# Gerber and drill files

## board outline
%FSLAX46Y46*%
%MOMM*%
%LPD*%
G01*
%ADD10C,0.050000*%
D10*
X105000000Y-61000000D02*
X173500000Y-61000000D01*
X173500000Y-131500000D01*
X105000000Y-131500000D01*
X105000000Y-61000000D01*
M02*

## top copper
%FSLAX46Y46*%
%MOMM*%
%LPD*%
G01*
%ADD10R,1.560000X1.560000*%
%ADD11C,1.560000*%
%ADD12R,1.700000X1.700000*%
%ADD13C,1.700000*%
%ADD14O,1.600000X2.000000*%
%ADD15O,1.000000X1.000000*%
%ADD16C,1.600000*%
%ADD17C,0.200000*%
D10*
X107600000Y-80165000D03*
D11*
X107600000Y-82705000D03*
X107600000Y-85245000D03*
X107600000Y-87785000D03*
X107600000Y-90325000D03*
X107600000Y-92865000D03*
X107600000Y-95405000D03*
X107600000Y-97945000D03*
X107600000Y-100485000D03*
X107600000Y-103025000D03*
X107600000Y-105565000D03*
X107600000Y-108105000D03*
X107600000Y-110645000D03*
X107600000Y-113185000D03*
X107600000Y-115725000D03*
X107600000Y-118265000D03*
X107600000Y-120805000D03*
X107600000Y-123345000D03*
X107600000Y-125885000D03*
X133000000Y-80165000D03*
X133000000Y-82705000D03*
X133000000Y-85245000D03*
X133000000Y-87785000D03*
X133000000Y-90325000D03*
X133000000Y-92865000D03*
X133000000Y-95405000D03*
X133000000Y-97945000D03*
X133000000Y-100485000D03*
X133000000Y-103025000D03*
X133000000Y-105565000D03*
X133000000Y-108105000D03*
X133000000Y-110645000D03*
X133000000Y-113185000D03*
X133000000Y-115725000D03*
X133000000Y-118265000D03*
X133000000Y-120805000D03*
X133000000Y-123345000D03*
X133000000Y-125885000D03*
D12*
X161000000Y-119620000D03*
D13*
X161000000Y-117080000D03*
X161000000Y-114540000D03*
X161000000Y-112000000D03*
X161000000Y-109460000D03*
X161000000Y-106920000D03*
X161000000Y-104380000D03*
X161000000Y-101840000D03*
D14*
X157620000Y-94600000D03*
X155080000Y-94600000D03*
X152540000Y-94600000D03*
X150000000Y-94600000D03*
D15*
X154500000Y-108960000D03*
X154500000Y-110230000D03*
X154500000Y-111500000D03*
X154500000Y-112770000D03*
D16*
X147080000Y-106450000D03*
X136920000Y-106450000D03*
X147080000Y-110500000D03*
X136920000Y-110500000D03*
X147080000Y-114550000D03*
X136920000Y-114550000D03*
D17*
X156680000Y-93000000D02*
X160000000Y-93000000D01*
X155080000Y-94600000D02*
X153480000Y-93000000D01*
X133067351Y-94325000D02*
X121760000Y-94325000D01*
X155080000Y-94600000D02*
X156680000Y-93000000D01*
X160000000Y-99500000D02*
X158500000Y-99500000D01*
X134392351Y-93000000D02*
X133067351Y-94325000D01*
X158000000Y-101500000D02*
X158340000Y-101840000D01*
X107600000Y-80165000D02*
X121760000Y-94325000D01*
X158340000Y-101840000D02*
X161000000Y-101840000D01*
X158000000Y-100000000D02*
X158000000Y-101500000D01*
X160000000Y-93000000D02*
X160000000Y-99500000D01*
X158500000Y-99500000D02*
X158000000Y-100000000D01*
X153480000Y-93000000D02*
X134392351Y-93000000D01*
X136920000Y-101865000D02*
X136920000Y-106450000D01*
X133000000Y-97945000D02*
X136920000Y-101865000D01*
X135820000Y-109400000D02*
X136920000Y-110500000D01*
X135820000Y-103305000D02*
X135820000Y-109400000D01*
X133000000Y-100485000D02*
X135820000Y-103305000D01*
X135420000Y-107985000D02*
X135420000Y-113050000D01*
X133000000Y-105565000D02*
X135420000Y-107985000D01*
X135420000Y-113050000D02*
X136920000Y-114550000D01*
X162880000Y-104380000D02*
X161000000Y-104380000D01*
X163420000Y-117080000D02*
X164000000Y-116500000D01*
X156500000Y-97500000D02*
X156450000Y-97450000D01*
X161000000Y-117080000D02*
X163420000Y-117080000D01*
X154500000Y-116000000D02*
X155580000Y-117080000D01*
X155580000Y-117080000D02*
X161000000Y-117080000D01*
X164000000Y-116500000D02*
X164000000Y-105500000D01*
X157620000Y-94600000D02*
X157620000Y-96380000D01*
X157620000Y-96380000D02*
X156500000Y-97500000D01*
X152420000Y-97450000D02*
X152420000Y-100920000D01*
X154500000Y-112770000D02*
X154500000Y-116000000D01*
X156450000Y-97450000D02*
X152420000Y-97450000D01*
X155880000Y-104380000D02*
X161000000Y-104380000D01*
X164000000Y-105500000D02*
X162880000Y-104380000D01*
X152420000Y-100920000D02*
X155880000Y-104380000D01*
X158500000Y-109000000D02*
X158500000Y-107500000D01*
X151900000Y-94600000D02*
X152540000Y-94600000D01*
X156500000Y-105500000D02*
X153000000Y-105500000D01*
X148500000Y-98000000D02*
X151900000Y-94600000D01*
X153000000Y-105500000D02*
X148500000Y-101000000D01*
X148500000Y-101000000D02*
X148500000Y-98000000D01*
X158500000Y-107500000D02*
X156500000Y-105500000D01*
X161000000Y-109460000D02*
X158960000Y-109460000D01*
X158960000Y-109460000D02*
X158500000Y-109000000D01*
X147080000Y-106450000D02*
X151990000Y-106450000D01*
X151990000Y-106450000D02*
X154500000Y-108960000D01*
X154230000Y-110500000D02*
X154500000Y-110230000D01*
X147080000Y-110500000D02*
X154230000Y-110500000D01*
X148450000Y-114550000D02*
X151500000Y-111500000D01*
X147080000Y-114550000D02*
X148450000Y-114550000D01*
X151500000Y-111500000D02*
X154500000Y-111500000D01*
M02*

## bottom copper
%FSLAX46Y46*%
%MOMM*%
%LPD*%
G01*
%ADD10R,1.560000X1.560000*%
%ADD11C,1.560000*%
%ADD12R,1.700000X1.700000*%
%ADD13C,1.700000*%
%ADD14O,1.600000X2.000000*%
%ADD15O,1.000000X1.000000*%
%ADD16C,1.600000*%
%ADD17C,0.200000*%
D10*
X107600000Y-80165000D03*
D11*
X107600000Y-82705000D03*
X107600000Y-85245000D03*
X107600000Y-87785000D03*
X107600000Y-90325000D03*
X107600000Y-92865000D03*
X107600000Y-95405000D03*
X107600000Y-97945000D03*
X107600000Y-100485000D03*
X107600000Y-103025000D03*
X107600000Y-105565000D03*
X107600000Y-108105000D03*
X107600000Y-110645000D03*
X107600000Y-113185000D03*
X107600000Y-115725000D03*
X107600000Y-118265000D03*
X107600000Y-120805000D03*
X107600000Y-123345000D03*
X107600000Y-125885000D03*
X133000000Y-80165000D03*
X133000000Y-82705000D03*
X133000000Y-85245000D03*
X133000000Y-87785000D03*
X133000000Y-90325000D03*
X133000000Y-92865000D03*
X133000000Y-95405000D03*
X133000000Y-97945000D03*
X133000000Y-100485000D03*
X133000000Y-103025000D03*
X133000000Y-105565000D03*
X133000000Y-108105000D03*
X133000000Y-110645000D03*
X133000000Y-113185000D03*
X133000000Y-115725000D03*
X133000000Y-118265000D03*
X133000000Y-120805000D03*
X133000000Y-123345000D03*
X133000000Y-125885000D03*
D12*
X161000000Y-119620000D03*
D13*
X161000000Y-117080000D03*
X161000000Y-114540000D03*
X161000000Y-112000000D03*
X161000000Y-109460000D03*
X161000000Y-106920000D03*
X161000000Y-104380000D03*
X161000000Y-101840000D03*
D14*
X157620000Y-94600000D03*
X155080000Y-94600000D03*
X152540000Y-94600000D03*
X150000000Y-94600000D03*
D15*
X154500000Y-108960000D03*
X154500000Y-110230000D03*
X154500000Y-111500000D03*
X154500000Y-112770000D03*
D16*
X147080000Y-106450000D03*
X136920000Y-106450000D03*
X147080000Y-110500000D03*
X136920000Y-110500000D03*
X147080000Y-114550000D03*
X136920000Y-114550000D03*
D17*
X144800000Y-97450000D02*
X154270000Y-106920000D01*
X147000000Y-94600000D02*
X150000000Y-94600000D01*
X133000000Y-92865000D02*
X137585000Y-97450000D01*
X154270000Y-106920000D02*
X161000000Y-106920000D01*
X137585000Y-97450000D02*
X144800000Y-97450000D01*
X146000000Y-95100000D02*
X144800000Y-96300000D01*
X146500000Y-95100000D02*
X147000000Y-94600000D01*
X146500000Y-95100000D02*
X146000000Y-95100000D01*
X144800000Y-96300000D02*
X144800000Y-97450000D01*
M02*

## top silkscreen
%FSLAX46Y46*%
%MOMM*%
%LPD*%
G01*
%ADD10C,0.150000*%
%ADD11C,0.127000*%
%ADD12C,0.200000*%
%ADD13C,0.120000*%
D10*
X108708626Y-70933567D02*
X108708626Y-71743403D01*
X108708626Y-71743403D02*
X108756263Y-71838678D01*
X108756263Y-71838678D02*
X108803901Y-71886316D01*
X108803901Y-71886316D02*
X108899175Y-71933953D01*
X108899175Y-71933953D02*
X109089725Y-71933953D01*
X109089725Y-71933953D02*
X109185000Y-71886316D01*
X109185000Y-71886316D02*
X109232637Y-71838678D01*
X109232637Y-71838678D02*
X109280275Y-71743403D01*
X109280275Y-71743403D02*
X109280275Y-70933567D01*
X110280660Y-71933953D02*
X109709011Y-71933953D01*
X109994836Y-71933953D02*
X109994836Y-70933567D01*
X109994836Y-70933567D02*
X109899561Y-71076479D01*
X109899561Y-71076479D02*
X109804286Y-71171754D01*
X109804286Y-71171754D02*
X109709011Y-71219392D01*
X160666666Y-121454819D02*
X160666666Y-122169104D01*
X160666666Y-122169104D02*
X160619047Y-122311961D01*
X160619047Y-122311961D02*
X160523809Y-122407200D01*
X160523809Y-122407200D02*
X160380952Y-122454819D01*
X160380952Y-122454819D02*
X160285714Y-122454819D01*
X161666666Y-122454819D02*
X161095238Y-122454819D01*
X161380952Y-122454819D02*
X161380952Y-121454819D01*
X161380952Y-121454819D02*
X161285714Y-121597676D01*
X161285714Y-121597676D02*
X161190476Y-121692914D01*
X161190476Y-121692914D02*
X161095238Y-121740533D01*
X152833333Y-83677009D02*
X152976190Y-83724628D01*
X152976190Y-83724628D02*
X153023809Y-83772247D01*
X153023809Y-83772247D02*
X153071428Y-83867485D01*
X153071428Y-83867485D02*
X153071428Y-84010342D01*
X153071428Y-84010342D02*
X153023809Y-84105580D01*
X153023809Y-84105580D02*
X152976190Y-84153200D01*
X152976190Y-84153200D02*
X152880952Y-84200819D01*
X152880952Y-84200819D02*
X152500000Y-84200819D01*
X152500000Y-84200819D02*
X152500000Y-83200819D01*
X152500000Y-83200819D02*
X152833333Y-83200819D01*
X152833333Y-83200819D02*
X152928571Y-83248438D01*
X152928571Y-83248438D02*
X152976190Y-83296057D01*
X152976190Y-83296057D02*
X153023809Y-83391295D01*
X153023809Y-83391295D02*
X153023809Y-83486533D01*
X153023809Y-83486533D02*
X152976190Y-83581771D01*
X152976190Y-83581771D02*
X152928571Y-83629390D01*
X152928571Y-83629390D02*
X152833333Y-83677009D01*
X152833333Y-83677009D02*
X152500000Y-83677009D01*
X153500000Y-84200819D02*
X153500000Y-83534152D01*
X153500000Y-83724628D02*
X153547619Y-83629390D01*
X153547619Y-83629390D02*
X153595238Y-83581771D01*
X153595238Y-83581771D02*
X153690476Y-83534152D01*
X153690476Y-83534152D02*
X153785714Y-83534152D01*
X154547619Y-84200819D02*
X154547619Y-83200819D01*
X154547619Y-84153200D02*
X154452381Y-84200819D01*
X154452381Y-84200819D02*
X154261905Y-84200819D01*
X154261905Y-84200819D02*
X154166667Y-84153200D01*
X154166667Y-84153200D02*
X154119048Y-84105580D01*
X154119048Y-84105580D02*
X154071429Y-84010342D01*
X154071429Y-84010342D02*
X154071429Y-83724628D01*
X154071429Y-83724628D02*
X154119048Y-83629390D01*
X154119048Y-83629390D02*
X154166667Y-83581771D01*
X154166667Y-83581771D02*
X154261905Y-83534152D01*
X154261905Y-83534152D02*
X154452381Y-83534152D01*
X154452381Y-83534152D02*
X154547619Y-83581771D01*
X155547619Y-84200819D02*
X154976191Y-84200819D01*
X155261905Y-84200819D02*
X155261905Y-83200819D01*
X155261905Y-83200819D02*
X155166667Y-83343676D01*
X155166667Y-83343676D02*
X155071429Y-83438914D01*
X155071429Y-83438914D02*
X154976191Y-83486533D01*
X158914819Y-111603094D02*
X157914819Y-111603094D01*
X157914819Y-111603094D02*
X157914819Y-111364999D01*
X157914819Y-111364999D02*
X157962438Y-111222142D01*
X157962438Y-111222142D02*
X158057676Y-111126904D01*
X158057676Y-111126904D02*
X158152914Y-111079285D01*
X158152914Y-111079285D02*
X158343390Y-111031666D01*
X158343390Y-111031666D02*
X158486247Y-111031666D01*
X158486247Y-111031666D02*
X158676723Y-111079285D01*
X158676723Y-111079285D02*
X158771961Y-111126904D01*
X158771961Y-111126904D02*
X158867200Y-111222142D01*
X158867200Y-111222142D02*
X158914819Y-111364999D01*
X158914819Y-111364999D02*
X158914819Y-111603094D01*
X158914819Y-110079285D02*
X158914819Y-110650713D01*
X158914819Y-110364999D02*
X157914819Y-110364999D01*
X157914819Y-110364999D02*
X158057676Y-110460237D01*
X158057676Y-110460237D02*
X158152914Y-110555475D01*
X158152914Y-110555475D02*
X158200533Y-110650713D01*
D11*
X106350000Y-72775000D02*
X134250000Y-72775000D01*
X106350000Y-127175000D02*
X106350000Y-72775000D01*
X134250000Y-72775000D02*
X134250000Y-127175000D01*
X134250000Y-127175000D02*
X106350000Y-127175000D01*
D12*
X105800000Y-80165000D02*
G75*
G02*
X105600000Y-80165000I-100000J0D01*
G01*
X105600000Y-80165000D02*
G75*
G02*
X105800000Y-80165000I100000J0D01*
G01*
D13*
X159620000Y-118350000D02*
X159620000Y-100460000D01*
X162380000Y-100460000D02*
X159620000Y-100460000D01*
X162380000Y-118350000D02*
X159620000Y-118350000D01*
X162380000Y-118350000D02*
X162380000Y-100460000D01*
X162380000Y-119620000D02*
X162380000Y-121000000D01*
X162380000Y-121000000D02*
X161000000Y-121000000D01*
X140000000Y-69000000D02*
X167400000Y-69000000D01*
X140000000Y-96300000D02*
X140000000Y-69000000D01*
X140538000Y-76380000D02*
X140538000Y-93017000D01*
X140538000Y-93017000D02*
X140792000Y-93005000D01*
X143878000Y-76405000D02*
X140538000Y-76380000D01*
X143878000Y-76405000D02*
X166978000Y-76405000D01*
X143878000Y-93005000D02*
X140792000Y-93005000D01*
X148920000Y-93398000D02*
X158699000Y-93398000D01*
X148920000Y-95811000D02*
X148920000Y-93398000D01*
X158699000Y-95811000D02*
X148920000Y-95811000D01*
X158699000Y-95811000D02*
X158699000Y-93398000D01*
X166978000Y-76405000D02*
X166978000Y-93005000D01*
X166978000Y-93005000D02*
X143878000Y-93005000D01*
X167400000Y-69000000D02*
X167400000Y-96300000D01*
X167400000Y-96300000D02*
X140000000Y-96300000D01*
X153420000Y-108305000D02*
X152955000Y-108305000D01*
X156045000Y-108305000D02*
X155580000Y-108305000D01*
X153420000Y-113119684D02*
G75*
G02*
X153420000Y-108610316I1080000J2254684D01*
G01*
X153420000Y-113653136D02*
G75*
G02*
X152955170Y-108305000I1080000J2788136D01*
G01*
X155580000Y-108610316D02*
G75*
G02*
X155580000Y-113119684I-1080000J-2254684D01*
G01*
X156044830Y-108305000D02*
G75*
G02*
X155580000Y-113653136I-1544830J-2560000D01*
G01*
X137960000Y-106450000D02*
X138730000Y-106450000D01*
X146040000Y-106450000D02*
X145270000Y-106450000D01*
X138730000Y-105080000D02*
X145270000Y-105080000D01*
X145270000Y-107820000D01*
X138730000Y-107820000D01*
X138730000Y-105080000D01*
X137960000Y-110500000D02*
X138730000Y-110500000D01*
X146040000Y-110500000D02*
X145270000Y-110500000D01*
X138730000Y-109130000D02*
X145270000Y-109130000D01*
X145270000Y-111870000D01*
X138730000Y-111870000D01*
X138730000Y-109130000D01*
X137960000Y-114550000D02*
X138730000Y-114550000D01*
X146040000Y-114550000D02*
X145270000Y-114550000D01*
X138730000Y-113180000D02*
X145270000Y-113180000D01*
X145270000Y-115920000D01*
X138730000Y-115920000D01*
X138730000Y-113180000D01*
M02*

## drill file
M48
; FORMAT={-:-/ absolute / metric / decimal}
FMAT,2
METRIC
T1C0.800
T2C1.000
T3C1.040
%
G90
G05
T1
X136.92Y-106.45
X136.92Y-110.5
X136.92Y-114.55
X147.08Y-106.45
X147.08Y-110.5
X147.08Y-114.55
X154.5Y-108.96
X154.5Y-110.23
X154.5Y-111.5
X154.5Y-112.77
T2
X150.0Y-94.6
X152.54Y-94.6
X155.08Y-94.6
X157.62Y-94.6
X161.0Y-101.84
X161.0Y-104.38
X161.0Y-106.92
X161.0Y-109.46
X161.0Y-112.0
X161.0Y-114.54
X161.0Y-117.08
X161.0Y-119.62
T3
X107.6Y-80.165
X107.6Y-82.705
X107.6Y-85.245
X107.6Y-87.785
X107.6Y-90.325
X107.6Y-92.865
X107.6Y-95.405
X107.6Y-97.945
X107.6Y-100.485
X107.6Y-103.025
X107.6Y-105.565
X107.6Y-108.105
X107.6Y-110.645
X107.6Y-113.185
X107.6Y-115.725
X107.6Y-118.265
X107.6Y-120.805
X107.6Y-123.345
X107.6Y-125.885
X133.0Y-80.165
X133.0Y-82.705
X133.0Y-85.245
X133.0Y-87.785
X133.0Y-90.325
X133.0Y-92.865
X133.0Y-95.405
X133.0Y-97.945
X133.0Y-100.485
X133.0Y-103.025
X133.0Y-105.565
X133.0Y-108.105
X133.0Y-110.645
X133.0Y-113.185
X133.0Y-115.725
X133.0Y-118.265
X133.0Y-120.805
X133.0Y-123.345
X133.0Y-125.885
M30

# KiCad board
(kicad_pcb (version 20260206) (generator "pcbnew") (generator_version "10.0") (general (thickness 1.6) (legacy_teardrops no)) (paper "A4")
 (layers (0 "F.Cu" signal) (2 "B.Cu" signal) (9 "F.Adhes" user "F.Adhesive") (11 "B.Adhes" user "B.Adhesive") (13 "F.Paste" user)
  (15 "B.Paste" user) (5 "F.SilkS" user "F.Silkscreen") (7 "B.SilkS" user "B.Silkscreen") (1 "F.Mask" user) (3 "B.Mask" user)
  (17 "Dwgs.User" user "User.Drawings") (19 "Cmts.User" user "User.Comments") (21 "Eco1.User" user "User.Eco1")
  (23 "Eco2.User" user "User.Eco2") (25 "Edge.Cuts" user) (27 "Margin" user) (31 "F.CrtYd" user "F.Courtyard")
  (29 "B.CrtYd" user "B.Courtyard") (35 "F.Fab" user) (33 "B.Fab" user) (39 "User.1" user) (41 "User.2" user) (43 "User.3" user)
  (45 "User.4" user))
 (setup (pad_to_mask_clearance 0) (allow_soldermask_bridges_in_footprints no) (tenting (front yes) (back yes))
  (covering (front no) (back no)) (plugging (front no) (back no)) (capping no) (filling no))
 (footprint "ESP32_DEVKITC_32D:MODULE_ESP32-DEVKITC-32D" (layer "F.Cu") (at 120.3 99.925)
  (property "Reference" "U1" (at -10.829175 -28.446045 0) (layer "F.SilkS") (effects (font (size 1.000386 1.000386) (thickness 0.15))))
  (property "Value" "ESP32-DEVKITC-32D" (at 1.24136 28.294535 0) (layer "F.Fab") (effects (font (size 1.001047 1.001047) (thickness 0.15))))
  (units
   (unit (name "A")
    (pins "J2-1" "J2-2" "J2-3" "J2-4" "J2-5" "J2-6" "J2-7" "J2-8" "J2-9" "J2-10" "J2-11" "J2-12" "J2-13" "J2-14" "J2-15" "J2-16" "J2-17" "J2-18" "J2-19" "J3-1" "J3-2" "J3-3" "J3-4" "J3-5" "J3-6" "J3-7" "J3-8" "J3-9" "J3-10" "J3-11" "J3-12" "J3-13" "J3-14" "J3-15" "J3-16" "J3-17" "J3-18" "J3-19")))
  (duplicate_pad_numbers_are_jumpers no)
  (fp_line (start -13.95 -27.15) (end 13.95 -27.15) (stroke (width 0.127) (type solid)) (layer "F.SilkS"))
  (fp_line (start -13.95 27.25) (end -13.95 -27.15) (stroke (width 0.127) (type solid)) (layer "F.SilkS"))
  (fp_line (start 13.95 -27.15) (end 13.95 27.25) (stroke (width 0.127) (type solid)) (layer "F.SilkS"))
  (fp_line (start 13.95 27.25) (end -13.95 27.25) (stroke (width 0.127) (type solid)) (layer "F.SilkS"))
  (fp_circle (center -14.6 -19.76) (end -14.5 -19.76) (stroke (width 0.2) (type solid)) (fill no) (layer "F.SilkS"))
  (pad "J2-1" thru_hole rect (at -12.7 -19.76) (size 1.56 1.56) (drill 1.04) (layers "*.Cu" "*.Mask") (remove_unused_layers no)
   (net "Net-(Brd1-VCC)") (solder_mask_margin 0.102))
  (pad "J2-2" thru_hole circle (at -12.7 -17.22) (size 1.56 1.56) (drill 1.04) (layers "*.Cu" "*.Mask") (remove_unused_layers no)
   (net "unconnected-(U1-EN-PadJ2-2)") (solder_mask_margin 0.102))
  (pad "J2-3" thru_hole circle (at -12.7 -14.68) (size 1.56 1.56) (drill 1.04) (layers "*.Cu" "*.Mask") (remove_unused_layers no)
   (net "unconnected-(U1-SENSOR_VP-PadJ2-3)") (solder_mask_margin 0.102))
  (pad "J2-4" thru_hole circle (at -12.7 -12.14) (size 1.56 1.56) (drill 1.04) (layers "*.Cu" "*.Mask") (remove_unused_layers no)
   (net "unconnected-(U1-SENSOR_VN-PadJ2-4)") (solder_mask_margin 0.102))
  (pad "J2-5" thru_hole circle (at -12.7 -9.6) (size 1.56 1.56) (drill 1.04) (layers "*.Cu" "*.Mask") (remove_unused_layers no)
   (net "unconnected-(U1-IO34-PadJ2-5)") (solder_mask_margin 0.102))
  (pad "J2-6" thru_hole circle (at -12.7 -7.06) (size 1.56 1.56) (drill 1.04) (layers "*.Cu" "*.Mask") (remove_unused_layers no)
   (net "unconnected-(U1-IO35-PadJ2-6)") (solder_mask_margin 0.102))
  (pad "J2-7" thru_hole circle (at -12.7 -4.52) (size 1.56 1.56) (drill 1.04) (layers "*.Cu" "*.Mask") (remove_unused_layers no)
   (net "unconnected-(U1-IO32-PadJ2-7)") (solder_mask_margin 0.102))
  (pad "J2-8" thru_hole circle (at -12.7 -1.98) (size 1.56 1.56) (drill 1.04) (layers "*.Cu" "*.Mask") (remove_unused_layers no)
   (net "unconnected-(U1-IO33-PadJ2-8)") (solder_mask_margin 0.102))
  (pad "J2-9" thru_hole circle (at -12.7 0.56) (size 1.56 1.56) (drill 1.04) (layers "*.Cu" "*.Mask") (remove_unused_layers no)
   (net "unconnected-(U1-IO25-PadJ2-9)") (solder_mask_margin 0.102))
  (pad "J2-10" thru_hole circle (at -12.7 3.1) (size 1.56 1.56) (drill 1.04) (layers "*.Cu" "*.Mask") (remove_unused_layers no)
   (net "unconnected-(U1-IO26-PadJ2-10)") (solder_mask_margin 0.102))
  (pad "J2-11" thru_hole circle (at -12.7 5.64) (size 1.56 1.56) (drill 1.04) (layers "*.Cu" "*.Mask") (remove_unused_layers no)
   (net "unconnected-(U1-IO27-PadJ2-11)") (solder_mask_margin 0.102))
  (pad "J2-12" thru_hole circle (at -12.7 8.18) (size 1.56 1.56) (drill 1.04) (layers "*.Cu" "*.Mask") (remove_unused_layers no)
   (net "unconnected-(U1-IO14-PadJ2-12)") (solder_mask_margin 0.102))
  (pad "J2-13" thru_hole circle (at -12.7 10.72) (size 1.56 1.56) (drill 1.04) (layers "*.Cu" "*.Mask") (remove_unused_layers no)
   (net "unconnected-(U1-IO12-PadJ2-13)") (solder_mask_margin 0.102))
  (pad "J2-14" thru_hole circle (at -12.7 13.26) (size 1.56 1.56) (drill 1.04) (layers "*.Cu" "*.Mask") (remove_unused_layers no)
   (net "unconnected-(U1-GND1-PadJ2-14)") (solder_mask_margin 0.102))
  (pad "J2-15" thru_hole circle (at -12.7 15.8) (size 1.56 1.56) (drill 1.04) (layers "*.Cu" "*.Mask") (remove_unused_layers no)
   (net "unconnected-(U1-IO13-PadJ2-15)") (solder_mask_margin 0.102))
  (pad "J2-16" thru_hole circle (at -12.7 18.34) (size 1.56 1.56) (drill 1.04) (layers "*.Cu" "*.Mask") (remove_unused_layers no)
   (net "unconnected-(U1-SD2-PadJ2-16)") (solder_mask_margin 0.102))
  (pad "J2-17" thru_hole circle (at -12.7 20.88) (size 1.56 1.56) (drill 1.04) (layers "*.Cu" "*.Mask") (remove_unused_layers no)
   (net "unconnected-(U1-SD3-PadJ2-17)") (solder_mask_margin 0.102))
  (pad "J2-18" thru_hole circle (at -12.7 23.42) (size 1.56 1.56) (drill 1.04) (layers "*.Cu" "*.Mask") (remove_unused_layers no)
   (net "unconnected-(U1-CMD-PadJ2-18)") (solder_mask_margin 0.102))
  (pad "J2-19" thru_hole circle (at -12.7 25.96) (size 1.56 1.56) (drill 1.04) (layers "*.Cu" "*.Mask") (remove_unused_layers no)
   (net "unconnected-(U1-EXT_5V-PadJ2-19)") (solder_mask_margin 0.102))
  (pad "J3-1" thru_hole circle (at 12.7 -19.76) (size 1.56 1.56) (drill 1.04) (layers "*.Cu" "*.Mask") (remove_unused_layers no)
   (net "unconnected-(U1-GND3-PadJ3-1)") (solder_mask_margin 0.102))
  (pad "J3-2" thru_hole circle (at 12.7 -17.22) (size 1.56 1.56) (drill 1.04) (layers "*.Cu" "*.Mask") (remove_unused_layers no)
   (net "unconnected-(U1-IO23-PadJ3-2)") (solder_mask_margin 0.102))
  (pad "J3-3" thru_hole circle (at 12.7 -14.68) (size 1.56 1.56) (drill 1.04) (layers "*.Cu" "*.Mask") (remove_unused_layers no)
   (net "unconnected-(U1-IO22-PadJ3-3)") (solder_mask_margin 0.102))
  (pad "J3-4" thru_hole circle (at 12.7 -12.14) (size 1.56 1.56) (drill 1.04) (layers "*.Cu" "*.Mask") (remove_unused_layers no)
   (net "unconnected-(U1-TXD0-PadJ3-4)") (solder_mask_margin 0.102))
  (pad "J3-5" thru_hole circle (at 12.7 -9.6) (size 1.56 1.56) (drill 1.04) (layers "*.Cu" "*.Mask") (remove_unused_layers no)
   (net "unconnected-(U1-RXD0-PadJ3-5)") (solder_mask_margin 0.102))
  (pad "J3-6" thru_hole circle (at 12.7 -7.06) (size 1.56 1.56) (drill 1.04) (layers "*.Cu" "*.Mask") (remove_unused_layers no) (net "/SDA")
   (solder_mask_margin 0.102))
  (pad "J3-7" thru_hole circle (at 12.7 -4.52) (size 1.56 1.56) (drill 1.04) (layers "*.Cu" "*.Mask") (remove_unused_layers no)
   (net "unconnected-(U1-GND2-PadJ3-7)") (solder_mask_margin 0.102))
  (pad "J3-8" thru_hole circle (at 12.7 -1.98) (size 1.56 1.56) (drill 1.04) (layers "*.Cu" "*.Mask") (remove_unused_layers no)
   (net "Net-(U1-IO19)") (solder_mask_margin 0.102))
  (pad "J3-9" thru_hole circle (at 12.7 0.56) (size 1.56 1.56) (drill 1.04) (layers "*.Cu" "*.Mask") (remove_unused_layers no)
   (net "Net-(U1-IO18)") (solder_mask_margin 0.102))
  (pad "J3-10" thru_hole circle (at 12.7 3.1) (size 1.56 1.56) (drill 1.04) (layers "*.Cu" "*.Mask") (remove_unused_layers no)
   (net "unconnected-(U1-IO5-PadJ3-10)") (solder_mask_margin 0.102))
  (pad "J3-11" thru_hole circle (at 12.7 5.64) (size 1.56 1.56) (drill 1.04) (layers "*.Cu" "*.Mask") (remove_unused_layers no)
   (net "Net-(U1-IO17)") (solder_mask_margin 0.102))
  (pad "J3-12" thru_hole circle (at 12.7 8.18) (size 1.56 1.56) (drill 1.04) (layers "*.Cu" "*.Mask") (remove_unused_layers no)
   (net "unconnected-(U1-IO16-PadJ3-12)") (solder_mask_margin 0.102))
  (pad "J3-13" thru_hole circle (at 12.7 10.72) (size 1.56 1.56) (drill 1.04) (layers "*.Cu" "*.Mask") (remove_unused_layers no)
   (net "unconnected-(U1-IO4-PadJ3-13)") (solder_mask_margin 0.102))
  (pad "J3-14" thru_hole circle (at 12.7 13.26) (size 1.56 1.56) (drill 1.04) (layers "*.Cu" "*.Mask") (remove_unused_layers no)
   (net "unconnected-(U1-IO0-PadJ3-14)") (solder_mask_margin 0.102))
  (pad "J3-15" thru_hole circle (at 12.7 15.8) (size 1.56 1.56) (drill 1.04) (layers "*.Cu" "*.Mask") (remove_unused_layers no)
   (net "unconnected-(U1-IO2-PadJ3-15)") (solder_mask_margin 0.102))
  (pad "J3-16" thru_hole circle (at 12.7 18.34) (size 1.56 1.56) (drill 1.04) (layers "*.Cu" "*.Mask") (remove_unused_layers no)
   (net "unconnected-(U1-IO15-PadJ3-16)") (solder_mask_margin 0.102))
  (pad "J3-17" thru_hole circle (at 12.7 20.88) (size 1.56 1.56) (drill 1.04) (layers "*.Cu" "*.Mask") (remove_unused_layers no)
   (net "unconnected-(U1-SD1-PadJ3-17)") (solder_mask_margin 0.102))
  (pad "J3-18" thru_hole circle (at 12.7 23.42) (size 1.56 1.56) (drill 1.04) (layers "*.Cu" "*.Mask") (remove_unused_layers no)
   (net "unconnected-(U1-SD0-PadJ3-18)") (solder_mask_margin 0.102))
  (pad "J3-19" thru_hole circle (at 12.7 25.96) (size 1.56 1.56) (drill 1.04) (layers "*.Cu" "*.Mask") (remove_unused_layers no)
   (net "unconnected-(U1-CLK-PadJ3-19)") (solder_mask_margin 0.102)))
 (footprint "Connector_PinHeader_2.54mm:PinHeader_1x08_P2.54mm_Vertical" (layer "F.Cu") (at 161 119.62 180)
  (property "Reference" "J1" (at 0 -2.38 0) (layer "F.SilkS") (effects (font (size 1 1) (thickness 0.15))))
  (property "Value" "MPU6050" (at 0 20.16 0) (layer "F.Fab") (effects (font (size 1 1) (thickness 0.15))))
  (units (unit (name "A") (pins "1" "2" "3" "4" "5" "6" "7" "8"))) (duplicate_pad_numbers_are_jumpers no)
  (fp_line (start 1.38 1.27) (end 1.38 19.16) (stroke (width 0.12) (type solid)) (layer "F.SilkS"))
  (fp_line (start -1.38 19.16) (end 1.38 19.16) (stroke (width 0.12) (type solid)) (layer "F.SilkS"))
  (fp_line (start -1.38 1.27) (end 1.38 1.27) (stroke (width 0.12) (type solid)) (layer "F.SilkS"))
  (fp_line (start -1.38 1.27) (end -1.38 19.16) (stroke (width 0.12) (type solid)) (layer "F.SilkS"))
  (fp_line (start -1.38 0) (end -1.38 -1.38) (stroke (width 0.12) (type solid)) (layer "F.SilkS"))
  (fp_line (start -1.38 -1.38) (end 0 -1.38) (stroke (width 0.12) (type solid)) (layer "F.SilkS"))
  (pad "1" thru_hole rect (at 0 0 180) (size 1.7 1.7) (drill 1) (layers "*.Cu" "*.Mask") (remove_unused_layers no)
   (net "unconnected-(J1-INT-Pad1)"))
  (pad "2" thru_hole circle (at 0 2.54 180) (size 1.7 1.7) (drill 1) (layers "*.Cu" "*.Mask") (remove_unused_layers no) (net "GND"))
  (pad "3" thru_hole circle (at 0 5.08 180) (size 1.7 1.7) (drill 1) (layers "*.Cu" "*.Mask") (remove_unused_layers no)
   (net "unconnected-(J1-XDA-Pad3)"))
  (pad "4" thru_hole circle (at 0 7.62 180) (size 1.7 1.7) (drill 1) (layers "*.Cu" "*.Mask") (remove_unused_layers no)
   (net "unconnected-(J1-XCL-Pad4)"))
  (pad "5" thru_hole circle (at 0 10.16 180) (size 1.7 1.7) (drill 1) (layers "*.Cu" "*.Mask") (remove_unused_layers no) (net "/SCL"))
  (pad "6" thru_hole circle (at 0 12.7 180) (size 1.7 1.7) (drill 1) (layers "*.Cu" "*.Mask") (remove_unused_layers no) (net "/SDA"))
  (pad "7" thru_hole circle (at 0 15.24 180) (size 1.7 1.7) (drill 1) (layers "*.Cu" "*.Mask") (remove_unused_layers no) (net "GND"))
  (pad "8" thru_hole circle (at 0 17.78 180) (size 1.7 1.7) (drill 1) (layers "*.Cu" "*.Mask") (remove_unused_layers no)
   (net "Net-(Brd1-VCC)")))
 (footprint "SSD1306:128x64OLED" (layer "F.Cu") (at 154 84 180)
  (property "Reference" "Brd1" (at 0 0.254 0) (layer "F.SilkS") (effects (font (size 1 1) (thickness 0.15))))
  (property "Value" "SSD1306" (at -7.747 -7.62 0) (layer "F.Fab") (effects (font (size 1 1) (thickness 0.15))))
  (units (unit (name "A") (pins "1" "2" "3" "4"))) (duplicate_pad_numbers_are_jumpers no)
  (fp_line (start 14 15) (end -13.4 15) (stroke (width 0.12) (type solid)) (layer "F.SilkS"))
  (fp_line (start 14 -12.3) (end 14 15) (stroke (width 0.12) (type solid)) (layer "F.SilkS"))
  (fp_line (start 13.462 7.62) (end 13.462 -9.017) (stroke (width 0.12) (type solid)) (layer "F.SilkS"))
  (fp_line (start 13.462 -9.017) (end 13.208 -9.005) (stroke (width 0.12) (type solid)) (layer "F.SilkS"))
  (fp_line (start 10.122 7.595) (end 13.462 7.62) (stroke (width 0.12) (type solid)) (layer "F.SilkS"))
  (fp_line (start 10.122 7.595) (end -12.978 7.595) (stroke (width 0.12) (type solid)) (layer "F.SilkS"))
  (fp_line (start 10.122 -9.005) (end 13.208 -9.005) (stroke (width 0.12) (type solid)) (layer "F.SilkS"))
  (fp_line (start 5.08 -9.398) (end -4.699 -9.398) (stroke (width 0.12) (type solid)) (layer "F.SilkS"))
  (fp_line (start 5.08 -11.811) (end 5.08 -9.398) (stroke (width 0.12) (type solid)) (layer "F.SilkS"))
  (fp_line (start -4.699 -11.811) (end 5.08 -11.811) (stroke (width 0.12) (type solid)) (layer "F.SilkS"))
  (fp_line (start -4.699 -11.811) (end -4.699 -9.398) (stroke (width 0.12) (type solid)) (layer "F.SilkS"))
  (fp_line (start -12.978 7.595) (end -12.978 -9.005) (stroke (width 0.12) (type solid)) (layer "F.SilkS"))
  (fp_line (start -12.978 -9.005) (end 10.122 -9.005) (stroke (width 0.12) (type solid)) (layer "F.SilkS"))
  (fp_line (start -13.4 15) (end -13.4 -12.3) (stroke (width 0.12) (type solid)) (layer "F.SilkS"))
  (fp_line (start -13.4 -12.3) (end 14 -12.3) (stroke (width 0.12) (type solid)) (layer "F.SilkS"))
  (pad "1" thru_hole oval (at -3.62 -10.6 270) (size 2 1.6) (drill 1) (layers "*.Cu" "*.Mask") (remove_unused_layers no) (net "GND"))
  (pad "2" thru_hole oval (at -1.08 -10.6 270) (size 2 1.6) (drill 1) (layers "*.Cu" "*.Mask") (remove_unused_layers no)
   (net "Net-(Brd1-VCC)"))
  (pad "3" thru_hole oval (at 1.46 -10.6 270) (size 2 1.6) (drill 1) (layers "*.Cu" "*.Mask") (remove_unused_layers no) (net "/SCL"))
  (pad "4" thru_hole oval (at 4 -10.6 270) (size 2 1.6) (drill 1) (layers "*.Cu" "*.Mask") (remove_unused_layers no) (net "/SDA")))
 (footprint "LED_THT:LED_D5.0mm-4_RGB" (layer "F.Cu") (at 154.5 108.96 -90)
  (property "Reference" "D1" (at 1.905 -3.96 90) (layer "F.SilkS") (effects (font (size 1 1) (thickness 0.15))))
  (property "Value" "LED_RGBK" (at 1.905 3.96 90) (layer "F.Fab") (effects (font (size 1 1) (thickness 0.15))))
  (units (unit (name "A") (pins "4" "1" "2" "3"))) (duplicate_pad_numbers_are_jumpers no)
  (fp_line (start -0.655 1.08) (end -0.655 1.545) (stroke (width 0.12) (type solid)) (layer "F.SilkS"))
  (fp_line (start -0.655 -1.545) (end -0.655 -1.08) (stroke (width 0.12) (type solid)) (layer "F.SilkS"))
  (fp_arc (start 4.159684 1.08) (mid 1.905 2.5) (end -0.349684 1.08) (stroke (width 0.12) (type solid)) (layer "F.SilkS"))
  (fp_arc (start 4.693136 1.08) (mid 2.163898 2.97877) (end -0.655 1.54483) (stroke (width 0.12) (type solid)) (layer "F.SilkS"))
  (fp_arc (start -0.349684 -1.08) (mid 1.905 -2.5) (end 4.159684 -1.08) (stroke (width 0.12) (type solid)) (layer "F.SilkS"))
  (fp_arc (start -0.655 -1.54483) (mid 2.163898 -2.97877) (end 4.693136 -1.08) (stroke (width 0.12) (type solid)) (layer "F.SilkS"))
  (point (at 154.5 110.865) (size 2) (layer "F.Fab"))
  (pad "1" thru_hole oval (at 0 0 270) (size 1 1) (drill 0.8) (layers "*.Cu" "*.Mask") (remove_unused_layers no) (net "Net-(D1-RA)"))
  (pad "2" thru_hole oval (at 1.27 0 270) (size 1 1) (drill 0.8) (layers "*.Cu" "*.Mask") (remove_unused_layers no) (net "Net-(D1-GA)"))
  (pad "3" thru_hole oval (at 2.54 0 270) (size 1 1) (drill 0.8) (layers "*.Cu" "*.Mask") (remove_unused_layers no) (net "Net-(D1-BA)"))
  (pad "4" thru_hole oval (at 3.81 0 270) (size 1 1) (drill 0.8) (layers "*.Cu" "*.Mask") (remove_unused_layers no) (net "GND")))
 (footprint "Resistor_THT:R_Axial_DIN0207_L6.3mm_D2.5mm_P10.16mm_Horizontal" (layer "F.Cu") (at 147.08 106.45 180)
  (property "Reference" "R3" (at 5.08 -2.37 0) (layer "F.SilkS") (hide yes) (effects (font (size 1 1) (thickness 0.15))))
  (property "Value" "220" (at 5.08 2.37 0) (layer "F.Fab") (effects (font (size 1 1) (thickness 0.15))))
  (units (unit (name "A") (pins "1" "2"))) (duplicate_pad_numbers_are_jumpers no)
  (fp_line (start 9.12 0) (end 8.35 0) (stroke (width 0.12) (type solid)) (layer "F.SilkS"))
  (fp_line (start 1.04 0) (end 1.81 0) (stroke (width 0.12) (type solid)) (layer "F.SilkS"))
  (fp_rect (start 1.81 -1.37) (end 8.35 1.37) (stroke (width 0.12) (type solid)) (fill no) (layer "F.SilkS"))
  (pad "1" thru_hole circle (at 0 0 180) (size 1.6 1.6) (drill 0.8) (layers "*.Cu" "*.Mask") (remove_unused_layers no) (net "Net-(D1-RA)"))
  (pad "2" thru_hole circle (at 10.16 0 180) (size 1.6 1.6) (drill 0.8) (layers "*.Cu" "*.Mask") (remove_unused_layers no)
   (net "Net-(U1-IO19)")))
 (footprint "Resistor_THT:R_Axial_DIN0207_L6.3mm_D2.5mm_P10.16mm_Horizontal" (layer "F.Cu") (at 147.08 110.5 180)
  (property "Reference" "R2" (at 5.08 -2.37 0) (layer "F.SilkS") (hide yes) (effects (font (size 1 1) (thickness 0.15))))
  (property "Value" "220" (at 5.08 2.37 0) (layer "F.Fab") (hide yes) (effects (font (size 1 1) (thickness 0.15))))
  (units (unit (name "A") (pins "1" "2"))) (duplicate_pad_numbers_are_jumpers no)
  (fp_line (start 9.12 0) (end 8.35 0) (stroke (width 0.12) (type solid)) (layer "F.SilkS"))
  (fp_line (start 1.04 0) (end 1.81 0) (stroke (width 0.12) (type solid)) (layer "F.SilkS"))
  (fp_rect (start 1.81 -1.37) (end 8.35 1.37) (stroke (width 0.12) (type solid)) (fill no) (layer "F.SilkS"))
  (pad "1" thru_hole circle (at 0 0 180) (size 1.6 1.6) (drill 0.8) (layers "*.Cu" "*.Mask") (remove_unused_layers no) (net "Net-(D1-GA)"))
  (pad "2" thru_hole circle (at 10.16 0 180) (size 1.6 1.6) (drill 0.8) (layers "*.Cu" "*.Mask") (remove_unused_layers no)
   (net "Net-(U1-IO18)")))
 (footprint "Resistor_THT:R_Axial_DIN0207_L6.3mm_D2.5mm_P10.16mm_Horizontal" (layer "F.Cu") (at 147.08 114.55 180)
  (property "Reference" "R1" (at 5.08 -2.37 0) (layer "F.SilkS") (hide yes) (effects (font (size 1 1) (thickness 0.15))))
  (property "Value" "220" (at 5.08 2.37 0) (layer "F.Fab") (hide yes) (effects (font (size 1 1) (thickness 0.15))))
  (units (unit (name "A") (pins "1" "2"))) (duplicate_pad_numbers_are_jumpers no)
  (fp_line (start 9.12 0) (end 8.35 0) (stroke (width 0.12) (type solid)) (layer "F.SilkS"))
  (fp_line (start 1.04 0) (end 1.81 0) (stroke (width 0.12) (type solid)) (layer "F.SilkS"))
  (fp_rect (start 1.81 -1.37) (end 8.35 1.37) (stroke (width 0.12) (type solid)) (fill no) (layer "F.SilkS"))
  (pad "1" thru_hole circle (at 0 0 180) (size 1.6 1.6) (drill 0.8) (layers "*.Cu" "*.Mask") (remove_unused_layers no) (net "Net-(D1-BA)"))
  (pad "2" thru_hole circle (at 10.16 0 180) (size 1.6 1.6) (drill 0.8) (layers "*.Cu" "*.Mask") (remove_unused_layers no)
   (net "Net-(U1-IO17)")))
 (gr_rect (start 105 61) (end 173.5 131.5) (stroke (width 0.05) (type default)) (fill no) (layer "Edge.Cuts"))
 (segment (start 156.68 93) (end 160 93) (width 0.2) (layer "F.Cu") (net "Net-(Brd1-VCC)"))
 (segment (start 155.08 94.6) (end 153.48 93) (width 0.2) (layer "F.Cu") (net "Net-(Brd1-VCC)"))
 (segment (start 133.067351 94.325) (end 121.76 94.325) (width 0.2) (layer "F.Cu") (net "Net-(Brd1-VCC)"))
 (segment (start 155.08 94.6) (end 156.68 93) (width 0.2) (layer "F.Cu") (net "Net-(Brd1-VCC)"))
 (segment (start 160 99.5) (end 158.5 99.5) (width 0.2) (layer "F.Cu") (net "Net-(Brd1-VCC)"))
 (segment (start 134.392351 93) (end 133.067351 94.325) (width 0.2) (layer "F.Cu") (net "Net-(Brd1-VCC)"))
 (segment (start 158 101.5) (end 158.34 101.84) (width 0.2) (layer "F.Cu") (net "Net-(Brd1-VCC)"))
 (segment (start 107.6 80.165) (end 121.76 94.325) (width 0.2) (layer "F.Cu") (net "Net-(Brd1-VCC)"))
 (segment (start 158.34 101.84) (end 161 101.84) (width 0.2) (layer "F.Cu") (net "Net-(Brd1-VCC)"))
 (segment (start 158 100) (end 158 101.5) (width 0.2) (layer "F.Cu") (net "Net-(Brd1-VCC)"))
 (segment (start 160 93) (end 160 99.5) (width 0.2) (layer "F.Cu") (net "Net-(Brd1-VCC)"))
 (segment (start 158.5 99.5) (end 158 100) (width 0.2) (layer "F.Cu") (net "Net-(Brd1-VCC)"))
 (segment (start 153.48 93) (end 134.392351 93) (width 0.2) (layer "F.Cu") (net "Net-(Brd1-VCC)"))
 (segment (start 144.8 97.45) (end 154.27 106.92) (width 0.2) (layer "B.Cu") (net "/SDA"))
 (segment (start 147 94.6) (end 150 94.6) (width 0.2) (layer "B.Cu") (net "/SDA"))
 (segment (start 133 92.865) (end 137.585 97.45) (width 0.2) (layer "B.Cu") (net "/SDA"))
 (segment (start 154.27 106.92) (end 161 106.92) (width 0.2) (layer "B.Cu") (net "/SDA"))
 (segment (start 137.585 97.45) (end 144.8 97.45) (width 0.2) (layer "B.Cu") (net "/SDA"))
 (segment (start 146 95.1) (end 144.8 96.3) (width 0.2) (layer "B.Cu") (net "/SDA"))
 (segment (start 146.5 95.1) (end 147 94.6) (width 0.2) (layer "B.Cu") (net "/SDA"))
 (segment (start 146.5 95.1) (end 146 95.1) (width 0.2) (layer "B.Cu") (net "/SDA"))
 (segment (start 144.8 96.3) (end 144.8 97.45) (width 0.2) (layer "B.Cu") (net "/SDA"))
 (segment (start 136.92 101.865) (end 136.92 106.45) (width 0.2) (layer "F.Cu") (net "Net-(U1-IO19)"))
 (segment (start 133 97.945) (end 136.92 101.865) (width 0.2) (layer "F.Cu") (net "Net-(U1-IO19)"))
 (segment (start 135.82 109.4) (end 136.92 110.5) (width 0.2) (layer "F.Cu") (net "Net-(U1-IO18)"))
 (segment (start 135.82 103.305) (end 135.82 109.4) (width 0.2) (layer "F.Cu") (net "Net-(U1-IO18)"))
 (segment (start 133 100.485) (end 135.82 103.305) (width 0.2) (layer "F.Cu") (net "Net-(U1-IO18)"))
 (segment (start 135.42 107.985) (end 135.42 113.05) (width 0.2) (layer "F.Cu") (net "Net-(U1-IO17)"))
 (segment (start 133 105.565) (end 135.42 107.985) (width 0.2) (layer "F.Cu") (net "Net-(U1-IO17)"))
 (segment (start 135.42 113.05) (end 136.92 114.55) (width 0.2) (layer "F.Cu") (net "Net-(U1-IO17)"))
 (segment (start 162.88 104.38) (end 161 104.38) (width 0.2) (layer "F.Cu") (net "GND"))
 (segment (start 163.42 117.08) (end 164 116.5) (width 0.2) (layer "F.Cu") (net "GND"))
 (segment (start 156.5 97.5) (end 156.45 97.45) (width 0.2) (layer "F.Cu") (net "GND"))
 (segment (start 161 117.08) (end 163.42 117.08) (width 0.2) (layer "F.Cu") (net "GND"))
 (segment (start 154.5 116) (end 155.58 117.08) (width 0.2) (layer "F.Cu") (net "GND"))
 (segment (start 155.58 117.08) (end 161 117.08) (width 0.2) (layer "F.Cu") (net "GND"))
 (segment (start 164 116.5) (end 164 105.5) (width 0.2) (layer "F.Cu") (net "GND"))
 (segment (start 157.62 94.6) (end 157.62 96.38) (width 0.2) (layer "F.Cu") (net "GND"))
 (segment (start 157.62 96.38) (end 156.5 97.5) (width 0.2) (layer "F.Cu") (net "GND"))
 (segment (start 152.42 97.45) (end 152.42 100.92) (width 0.2) (layer "F.Cu") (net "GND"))
 (segment (start 154.5 112.77) (end 154.5 116) (width 0.2) (layer "F.Cu") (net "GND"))
 (segment (start 156.45 97.45) (end 152.42 97.45) (width 0.2) (layer "F.Cu") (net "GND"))
 (segment (start 155.88 104.38) (end 161 104.38) (width 0.2) (layer "F.Cu") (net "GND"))
 (segment (start 164 105.5) (end 162.88 104.38) (width 0.2) (layer "F.Cu") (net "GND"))
 (segment (start 152.42 100.92) (end 155.88 104.38) (width 0.2) (layer "F.Cu") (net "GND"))
 (segment (start 158.5 109) (end 158.5 107.5) (width 0.2) (layer "F.Cu") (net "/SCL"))
 (segment (start 151.9 94.6) (end 152.54 94.6) (width 0.2) (layer "F.Cu") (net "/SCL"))
 (segment (start 156.5 105.5) (end 153 105.5) (width 0.2) (layer "F.Cu") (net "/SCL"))
 (segment (start 148.5 98) (end 151.9 94.6) (width 0.2) (layer "F.Cu") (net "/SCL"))
 (segment (start 153 105.5) (end 148.5 101) (width 0.2) (layer "F.Cu") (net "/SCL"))
 (segment (start 148.5 101) (end 148.5 98) (width 0.2) (layer "F.Cu") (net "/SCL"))
 (segment (start 158.5 107.5) (end 156.5 105.5) (width 0.2) (layer "F.Cu") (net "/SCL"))
 (segment (start 161 109.46) (end 158.96 109.46) (width 0.2) (layer "F.Cu") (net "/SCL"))
 (segment (start 158.96 109.46) (end 158.5 109) (width 0.2) (layer "F.Cu") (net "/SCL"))
 (segment (start 147.08 106.45) (end 151.99 106.45) (width 0.2) (layer "F.Cu") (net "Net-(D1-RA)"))
 (segment (start 151.99 106.45) (end 154.5 108.96) (width 0.2) (layer "F.Cu") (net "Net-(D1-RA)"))
 (segment (start 154.23 110.5) (end 154.5 110.23) (width 0.2) (layer "F.Cu") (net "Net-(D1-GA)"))
 (segment (start 147.08 110.5) (end 154.23 110.5) (width 0.2) (layer "F.Cu") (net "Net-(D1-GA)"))
 (segment (start 148.45 114.55) (end 151.5 111.5) (width 0.2) (layer "F.Cu") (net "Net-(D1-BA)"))
 (segment (start 147.08 114.55) (end 148.45 114.55) (width 0.2) (layer "F.Cu") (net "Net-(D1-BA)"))
 (segment (start 151.5 111.5) (end 154.5 111.5) (width 0.2) (layer "F.Cu") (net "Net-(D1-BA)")))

